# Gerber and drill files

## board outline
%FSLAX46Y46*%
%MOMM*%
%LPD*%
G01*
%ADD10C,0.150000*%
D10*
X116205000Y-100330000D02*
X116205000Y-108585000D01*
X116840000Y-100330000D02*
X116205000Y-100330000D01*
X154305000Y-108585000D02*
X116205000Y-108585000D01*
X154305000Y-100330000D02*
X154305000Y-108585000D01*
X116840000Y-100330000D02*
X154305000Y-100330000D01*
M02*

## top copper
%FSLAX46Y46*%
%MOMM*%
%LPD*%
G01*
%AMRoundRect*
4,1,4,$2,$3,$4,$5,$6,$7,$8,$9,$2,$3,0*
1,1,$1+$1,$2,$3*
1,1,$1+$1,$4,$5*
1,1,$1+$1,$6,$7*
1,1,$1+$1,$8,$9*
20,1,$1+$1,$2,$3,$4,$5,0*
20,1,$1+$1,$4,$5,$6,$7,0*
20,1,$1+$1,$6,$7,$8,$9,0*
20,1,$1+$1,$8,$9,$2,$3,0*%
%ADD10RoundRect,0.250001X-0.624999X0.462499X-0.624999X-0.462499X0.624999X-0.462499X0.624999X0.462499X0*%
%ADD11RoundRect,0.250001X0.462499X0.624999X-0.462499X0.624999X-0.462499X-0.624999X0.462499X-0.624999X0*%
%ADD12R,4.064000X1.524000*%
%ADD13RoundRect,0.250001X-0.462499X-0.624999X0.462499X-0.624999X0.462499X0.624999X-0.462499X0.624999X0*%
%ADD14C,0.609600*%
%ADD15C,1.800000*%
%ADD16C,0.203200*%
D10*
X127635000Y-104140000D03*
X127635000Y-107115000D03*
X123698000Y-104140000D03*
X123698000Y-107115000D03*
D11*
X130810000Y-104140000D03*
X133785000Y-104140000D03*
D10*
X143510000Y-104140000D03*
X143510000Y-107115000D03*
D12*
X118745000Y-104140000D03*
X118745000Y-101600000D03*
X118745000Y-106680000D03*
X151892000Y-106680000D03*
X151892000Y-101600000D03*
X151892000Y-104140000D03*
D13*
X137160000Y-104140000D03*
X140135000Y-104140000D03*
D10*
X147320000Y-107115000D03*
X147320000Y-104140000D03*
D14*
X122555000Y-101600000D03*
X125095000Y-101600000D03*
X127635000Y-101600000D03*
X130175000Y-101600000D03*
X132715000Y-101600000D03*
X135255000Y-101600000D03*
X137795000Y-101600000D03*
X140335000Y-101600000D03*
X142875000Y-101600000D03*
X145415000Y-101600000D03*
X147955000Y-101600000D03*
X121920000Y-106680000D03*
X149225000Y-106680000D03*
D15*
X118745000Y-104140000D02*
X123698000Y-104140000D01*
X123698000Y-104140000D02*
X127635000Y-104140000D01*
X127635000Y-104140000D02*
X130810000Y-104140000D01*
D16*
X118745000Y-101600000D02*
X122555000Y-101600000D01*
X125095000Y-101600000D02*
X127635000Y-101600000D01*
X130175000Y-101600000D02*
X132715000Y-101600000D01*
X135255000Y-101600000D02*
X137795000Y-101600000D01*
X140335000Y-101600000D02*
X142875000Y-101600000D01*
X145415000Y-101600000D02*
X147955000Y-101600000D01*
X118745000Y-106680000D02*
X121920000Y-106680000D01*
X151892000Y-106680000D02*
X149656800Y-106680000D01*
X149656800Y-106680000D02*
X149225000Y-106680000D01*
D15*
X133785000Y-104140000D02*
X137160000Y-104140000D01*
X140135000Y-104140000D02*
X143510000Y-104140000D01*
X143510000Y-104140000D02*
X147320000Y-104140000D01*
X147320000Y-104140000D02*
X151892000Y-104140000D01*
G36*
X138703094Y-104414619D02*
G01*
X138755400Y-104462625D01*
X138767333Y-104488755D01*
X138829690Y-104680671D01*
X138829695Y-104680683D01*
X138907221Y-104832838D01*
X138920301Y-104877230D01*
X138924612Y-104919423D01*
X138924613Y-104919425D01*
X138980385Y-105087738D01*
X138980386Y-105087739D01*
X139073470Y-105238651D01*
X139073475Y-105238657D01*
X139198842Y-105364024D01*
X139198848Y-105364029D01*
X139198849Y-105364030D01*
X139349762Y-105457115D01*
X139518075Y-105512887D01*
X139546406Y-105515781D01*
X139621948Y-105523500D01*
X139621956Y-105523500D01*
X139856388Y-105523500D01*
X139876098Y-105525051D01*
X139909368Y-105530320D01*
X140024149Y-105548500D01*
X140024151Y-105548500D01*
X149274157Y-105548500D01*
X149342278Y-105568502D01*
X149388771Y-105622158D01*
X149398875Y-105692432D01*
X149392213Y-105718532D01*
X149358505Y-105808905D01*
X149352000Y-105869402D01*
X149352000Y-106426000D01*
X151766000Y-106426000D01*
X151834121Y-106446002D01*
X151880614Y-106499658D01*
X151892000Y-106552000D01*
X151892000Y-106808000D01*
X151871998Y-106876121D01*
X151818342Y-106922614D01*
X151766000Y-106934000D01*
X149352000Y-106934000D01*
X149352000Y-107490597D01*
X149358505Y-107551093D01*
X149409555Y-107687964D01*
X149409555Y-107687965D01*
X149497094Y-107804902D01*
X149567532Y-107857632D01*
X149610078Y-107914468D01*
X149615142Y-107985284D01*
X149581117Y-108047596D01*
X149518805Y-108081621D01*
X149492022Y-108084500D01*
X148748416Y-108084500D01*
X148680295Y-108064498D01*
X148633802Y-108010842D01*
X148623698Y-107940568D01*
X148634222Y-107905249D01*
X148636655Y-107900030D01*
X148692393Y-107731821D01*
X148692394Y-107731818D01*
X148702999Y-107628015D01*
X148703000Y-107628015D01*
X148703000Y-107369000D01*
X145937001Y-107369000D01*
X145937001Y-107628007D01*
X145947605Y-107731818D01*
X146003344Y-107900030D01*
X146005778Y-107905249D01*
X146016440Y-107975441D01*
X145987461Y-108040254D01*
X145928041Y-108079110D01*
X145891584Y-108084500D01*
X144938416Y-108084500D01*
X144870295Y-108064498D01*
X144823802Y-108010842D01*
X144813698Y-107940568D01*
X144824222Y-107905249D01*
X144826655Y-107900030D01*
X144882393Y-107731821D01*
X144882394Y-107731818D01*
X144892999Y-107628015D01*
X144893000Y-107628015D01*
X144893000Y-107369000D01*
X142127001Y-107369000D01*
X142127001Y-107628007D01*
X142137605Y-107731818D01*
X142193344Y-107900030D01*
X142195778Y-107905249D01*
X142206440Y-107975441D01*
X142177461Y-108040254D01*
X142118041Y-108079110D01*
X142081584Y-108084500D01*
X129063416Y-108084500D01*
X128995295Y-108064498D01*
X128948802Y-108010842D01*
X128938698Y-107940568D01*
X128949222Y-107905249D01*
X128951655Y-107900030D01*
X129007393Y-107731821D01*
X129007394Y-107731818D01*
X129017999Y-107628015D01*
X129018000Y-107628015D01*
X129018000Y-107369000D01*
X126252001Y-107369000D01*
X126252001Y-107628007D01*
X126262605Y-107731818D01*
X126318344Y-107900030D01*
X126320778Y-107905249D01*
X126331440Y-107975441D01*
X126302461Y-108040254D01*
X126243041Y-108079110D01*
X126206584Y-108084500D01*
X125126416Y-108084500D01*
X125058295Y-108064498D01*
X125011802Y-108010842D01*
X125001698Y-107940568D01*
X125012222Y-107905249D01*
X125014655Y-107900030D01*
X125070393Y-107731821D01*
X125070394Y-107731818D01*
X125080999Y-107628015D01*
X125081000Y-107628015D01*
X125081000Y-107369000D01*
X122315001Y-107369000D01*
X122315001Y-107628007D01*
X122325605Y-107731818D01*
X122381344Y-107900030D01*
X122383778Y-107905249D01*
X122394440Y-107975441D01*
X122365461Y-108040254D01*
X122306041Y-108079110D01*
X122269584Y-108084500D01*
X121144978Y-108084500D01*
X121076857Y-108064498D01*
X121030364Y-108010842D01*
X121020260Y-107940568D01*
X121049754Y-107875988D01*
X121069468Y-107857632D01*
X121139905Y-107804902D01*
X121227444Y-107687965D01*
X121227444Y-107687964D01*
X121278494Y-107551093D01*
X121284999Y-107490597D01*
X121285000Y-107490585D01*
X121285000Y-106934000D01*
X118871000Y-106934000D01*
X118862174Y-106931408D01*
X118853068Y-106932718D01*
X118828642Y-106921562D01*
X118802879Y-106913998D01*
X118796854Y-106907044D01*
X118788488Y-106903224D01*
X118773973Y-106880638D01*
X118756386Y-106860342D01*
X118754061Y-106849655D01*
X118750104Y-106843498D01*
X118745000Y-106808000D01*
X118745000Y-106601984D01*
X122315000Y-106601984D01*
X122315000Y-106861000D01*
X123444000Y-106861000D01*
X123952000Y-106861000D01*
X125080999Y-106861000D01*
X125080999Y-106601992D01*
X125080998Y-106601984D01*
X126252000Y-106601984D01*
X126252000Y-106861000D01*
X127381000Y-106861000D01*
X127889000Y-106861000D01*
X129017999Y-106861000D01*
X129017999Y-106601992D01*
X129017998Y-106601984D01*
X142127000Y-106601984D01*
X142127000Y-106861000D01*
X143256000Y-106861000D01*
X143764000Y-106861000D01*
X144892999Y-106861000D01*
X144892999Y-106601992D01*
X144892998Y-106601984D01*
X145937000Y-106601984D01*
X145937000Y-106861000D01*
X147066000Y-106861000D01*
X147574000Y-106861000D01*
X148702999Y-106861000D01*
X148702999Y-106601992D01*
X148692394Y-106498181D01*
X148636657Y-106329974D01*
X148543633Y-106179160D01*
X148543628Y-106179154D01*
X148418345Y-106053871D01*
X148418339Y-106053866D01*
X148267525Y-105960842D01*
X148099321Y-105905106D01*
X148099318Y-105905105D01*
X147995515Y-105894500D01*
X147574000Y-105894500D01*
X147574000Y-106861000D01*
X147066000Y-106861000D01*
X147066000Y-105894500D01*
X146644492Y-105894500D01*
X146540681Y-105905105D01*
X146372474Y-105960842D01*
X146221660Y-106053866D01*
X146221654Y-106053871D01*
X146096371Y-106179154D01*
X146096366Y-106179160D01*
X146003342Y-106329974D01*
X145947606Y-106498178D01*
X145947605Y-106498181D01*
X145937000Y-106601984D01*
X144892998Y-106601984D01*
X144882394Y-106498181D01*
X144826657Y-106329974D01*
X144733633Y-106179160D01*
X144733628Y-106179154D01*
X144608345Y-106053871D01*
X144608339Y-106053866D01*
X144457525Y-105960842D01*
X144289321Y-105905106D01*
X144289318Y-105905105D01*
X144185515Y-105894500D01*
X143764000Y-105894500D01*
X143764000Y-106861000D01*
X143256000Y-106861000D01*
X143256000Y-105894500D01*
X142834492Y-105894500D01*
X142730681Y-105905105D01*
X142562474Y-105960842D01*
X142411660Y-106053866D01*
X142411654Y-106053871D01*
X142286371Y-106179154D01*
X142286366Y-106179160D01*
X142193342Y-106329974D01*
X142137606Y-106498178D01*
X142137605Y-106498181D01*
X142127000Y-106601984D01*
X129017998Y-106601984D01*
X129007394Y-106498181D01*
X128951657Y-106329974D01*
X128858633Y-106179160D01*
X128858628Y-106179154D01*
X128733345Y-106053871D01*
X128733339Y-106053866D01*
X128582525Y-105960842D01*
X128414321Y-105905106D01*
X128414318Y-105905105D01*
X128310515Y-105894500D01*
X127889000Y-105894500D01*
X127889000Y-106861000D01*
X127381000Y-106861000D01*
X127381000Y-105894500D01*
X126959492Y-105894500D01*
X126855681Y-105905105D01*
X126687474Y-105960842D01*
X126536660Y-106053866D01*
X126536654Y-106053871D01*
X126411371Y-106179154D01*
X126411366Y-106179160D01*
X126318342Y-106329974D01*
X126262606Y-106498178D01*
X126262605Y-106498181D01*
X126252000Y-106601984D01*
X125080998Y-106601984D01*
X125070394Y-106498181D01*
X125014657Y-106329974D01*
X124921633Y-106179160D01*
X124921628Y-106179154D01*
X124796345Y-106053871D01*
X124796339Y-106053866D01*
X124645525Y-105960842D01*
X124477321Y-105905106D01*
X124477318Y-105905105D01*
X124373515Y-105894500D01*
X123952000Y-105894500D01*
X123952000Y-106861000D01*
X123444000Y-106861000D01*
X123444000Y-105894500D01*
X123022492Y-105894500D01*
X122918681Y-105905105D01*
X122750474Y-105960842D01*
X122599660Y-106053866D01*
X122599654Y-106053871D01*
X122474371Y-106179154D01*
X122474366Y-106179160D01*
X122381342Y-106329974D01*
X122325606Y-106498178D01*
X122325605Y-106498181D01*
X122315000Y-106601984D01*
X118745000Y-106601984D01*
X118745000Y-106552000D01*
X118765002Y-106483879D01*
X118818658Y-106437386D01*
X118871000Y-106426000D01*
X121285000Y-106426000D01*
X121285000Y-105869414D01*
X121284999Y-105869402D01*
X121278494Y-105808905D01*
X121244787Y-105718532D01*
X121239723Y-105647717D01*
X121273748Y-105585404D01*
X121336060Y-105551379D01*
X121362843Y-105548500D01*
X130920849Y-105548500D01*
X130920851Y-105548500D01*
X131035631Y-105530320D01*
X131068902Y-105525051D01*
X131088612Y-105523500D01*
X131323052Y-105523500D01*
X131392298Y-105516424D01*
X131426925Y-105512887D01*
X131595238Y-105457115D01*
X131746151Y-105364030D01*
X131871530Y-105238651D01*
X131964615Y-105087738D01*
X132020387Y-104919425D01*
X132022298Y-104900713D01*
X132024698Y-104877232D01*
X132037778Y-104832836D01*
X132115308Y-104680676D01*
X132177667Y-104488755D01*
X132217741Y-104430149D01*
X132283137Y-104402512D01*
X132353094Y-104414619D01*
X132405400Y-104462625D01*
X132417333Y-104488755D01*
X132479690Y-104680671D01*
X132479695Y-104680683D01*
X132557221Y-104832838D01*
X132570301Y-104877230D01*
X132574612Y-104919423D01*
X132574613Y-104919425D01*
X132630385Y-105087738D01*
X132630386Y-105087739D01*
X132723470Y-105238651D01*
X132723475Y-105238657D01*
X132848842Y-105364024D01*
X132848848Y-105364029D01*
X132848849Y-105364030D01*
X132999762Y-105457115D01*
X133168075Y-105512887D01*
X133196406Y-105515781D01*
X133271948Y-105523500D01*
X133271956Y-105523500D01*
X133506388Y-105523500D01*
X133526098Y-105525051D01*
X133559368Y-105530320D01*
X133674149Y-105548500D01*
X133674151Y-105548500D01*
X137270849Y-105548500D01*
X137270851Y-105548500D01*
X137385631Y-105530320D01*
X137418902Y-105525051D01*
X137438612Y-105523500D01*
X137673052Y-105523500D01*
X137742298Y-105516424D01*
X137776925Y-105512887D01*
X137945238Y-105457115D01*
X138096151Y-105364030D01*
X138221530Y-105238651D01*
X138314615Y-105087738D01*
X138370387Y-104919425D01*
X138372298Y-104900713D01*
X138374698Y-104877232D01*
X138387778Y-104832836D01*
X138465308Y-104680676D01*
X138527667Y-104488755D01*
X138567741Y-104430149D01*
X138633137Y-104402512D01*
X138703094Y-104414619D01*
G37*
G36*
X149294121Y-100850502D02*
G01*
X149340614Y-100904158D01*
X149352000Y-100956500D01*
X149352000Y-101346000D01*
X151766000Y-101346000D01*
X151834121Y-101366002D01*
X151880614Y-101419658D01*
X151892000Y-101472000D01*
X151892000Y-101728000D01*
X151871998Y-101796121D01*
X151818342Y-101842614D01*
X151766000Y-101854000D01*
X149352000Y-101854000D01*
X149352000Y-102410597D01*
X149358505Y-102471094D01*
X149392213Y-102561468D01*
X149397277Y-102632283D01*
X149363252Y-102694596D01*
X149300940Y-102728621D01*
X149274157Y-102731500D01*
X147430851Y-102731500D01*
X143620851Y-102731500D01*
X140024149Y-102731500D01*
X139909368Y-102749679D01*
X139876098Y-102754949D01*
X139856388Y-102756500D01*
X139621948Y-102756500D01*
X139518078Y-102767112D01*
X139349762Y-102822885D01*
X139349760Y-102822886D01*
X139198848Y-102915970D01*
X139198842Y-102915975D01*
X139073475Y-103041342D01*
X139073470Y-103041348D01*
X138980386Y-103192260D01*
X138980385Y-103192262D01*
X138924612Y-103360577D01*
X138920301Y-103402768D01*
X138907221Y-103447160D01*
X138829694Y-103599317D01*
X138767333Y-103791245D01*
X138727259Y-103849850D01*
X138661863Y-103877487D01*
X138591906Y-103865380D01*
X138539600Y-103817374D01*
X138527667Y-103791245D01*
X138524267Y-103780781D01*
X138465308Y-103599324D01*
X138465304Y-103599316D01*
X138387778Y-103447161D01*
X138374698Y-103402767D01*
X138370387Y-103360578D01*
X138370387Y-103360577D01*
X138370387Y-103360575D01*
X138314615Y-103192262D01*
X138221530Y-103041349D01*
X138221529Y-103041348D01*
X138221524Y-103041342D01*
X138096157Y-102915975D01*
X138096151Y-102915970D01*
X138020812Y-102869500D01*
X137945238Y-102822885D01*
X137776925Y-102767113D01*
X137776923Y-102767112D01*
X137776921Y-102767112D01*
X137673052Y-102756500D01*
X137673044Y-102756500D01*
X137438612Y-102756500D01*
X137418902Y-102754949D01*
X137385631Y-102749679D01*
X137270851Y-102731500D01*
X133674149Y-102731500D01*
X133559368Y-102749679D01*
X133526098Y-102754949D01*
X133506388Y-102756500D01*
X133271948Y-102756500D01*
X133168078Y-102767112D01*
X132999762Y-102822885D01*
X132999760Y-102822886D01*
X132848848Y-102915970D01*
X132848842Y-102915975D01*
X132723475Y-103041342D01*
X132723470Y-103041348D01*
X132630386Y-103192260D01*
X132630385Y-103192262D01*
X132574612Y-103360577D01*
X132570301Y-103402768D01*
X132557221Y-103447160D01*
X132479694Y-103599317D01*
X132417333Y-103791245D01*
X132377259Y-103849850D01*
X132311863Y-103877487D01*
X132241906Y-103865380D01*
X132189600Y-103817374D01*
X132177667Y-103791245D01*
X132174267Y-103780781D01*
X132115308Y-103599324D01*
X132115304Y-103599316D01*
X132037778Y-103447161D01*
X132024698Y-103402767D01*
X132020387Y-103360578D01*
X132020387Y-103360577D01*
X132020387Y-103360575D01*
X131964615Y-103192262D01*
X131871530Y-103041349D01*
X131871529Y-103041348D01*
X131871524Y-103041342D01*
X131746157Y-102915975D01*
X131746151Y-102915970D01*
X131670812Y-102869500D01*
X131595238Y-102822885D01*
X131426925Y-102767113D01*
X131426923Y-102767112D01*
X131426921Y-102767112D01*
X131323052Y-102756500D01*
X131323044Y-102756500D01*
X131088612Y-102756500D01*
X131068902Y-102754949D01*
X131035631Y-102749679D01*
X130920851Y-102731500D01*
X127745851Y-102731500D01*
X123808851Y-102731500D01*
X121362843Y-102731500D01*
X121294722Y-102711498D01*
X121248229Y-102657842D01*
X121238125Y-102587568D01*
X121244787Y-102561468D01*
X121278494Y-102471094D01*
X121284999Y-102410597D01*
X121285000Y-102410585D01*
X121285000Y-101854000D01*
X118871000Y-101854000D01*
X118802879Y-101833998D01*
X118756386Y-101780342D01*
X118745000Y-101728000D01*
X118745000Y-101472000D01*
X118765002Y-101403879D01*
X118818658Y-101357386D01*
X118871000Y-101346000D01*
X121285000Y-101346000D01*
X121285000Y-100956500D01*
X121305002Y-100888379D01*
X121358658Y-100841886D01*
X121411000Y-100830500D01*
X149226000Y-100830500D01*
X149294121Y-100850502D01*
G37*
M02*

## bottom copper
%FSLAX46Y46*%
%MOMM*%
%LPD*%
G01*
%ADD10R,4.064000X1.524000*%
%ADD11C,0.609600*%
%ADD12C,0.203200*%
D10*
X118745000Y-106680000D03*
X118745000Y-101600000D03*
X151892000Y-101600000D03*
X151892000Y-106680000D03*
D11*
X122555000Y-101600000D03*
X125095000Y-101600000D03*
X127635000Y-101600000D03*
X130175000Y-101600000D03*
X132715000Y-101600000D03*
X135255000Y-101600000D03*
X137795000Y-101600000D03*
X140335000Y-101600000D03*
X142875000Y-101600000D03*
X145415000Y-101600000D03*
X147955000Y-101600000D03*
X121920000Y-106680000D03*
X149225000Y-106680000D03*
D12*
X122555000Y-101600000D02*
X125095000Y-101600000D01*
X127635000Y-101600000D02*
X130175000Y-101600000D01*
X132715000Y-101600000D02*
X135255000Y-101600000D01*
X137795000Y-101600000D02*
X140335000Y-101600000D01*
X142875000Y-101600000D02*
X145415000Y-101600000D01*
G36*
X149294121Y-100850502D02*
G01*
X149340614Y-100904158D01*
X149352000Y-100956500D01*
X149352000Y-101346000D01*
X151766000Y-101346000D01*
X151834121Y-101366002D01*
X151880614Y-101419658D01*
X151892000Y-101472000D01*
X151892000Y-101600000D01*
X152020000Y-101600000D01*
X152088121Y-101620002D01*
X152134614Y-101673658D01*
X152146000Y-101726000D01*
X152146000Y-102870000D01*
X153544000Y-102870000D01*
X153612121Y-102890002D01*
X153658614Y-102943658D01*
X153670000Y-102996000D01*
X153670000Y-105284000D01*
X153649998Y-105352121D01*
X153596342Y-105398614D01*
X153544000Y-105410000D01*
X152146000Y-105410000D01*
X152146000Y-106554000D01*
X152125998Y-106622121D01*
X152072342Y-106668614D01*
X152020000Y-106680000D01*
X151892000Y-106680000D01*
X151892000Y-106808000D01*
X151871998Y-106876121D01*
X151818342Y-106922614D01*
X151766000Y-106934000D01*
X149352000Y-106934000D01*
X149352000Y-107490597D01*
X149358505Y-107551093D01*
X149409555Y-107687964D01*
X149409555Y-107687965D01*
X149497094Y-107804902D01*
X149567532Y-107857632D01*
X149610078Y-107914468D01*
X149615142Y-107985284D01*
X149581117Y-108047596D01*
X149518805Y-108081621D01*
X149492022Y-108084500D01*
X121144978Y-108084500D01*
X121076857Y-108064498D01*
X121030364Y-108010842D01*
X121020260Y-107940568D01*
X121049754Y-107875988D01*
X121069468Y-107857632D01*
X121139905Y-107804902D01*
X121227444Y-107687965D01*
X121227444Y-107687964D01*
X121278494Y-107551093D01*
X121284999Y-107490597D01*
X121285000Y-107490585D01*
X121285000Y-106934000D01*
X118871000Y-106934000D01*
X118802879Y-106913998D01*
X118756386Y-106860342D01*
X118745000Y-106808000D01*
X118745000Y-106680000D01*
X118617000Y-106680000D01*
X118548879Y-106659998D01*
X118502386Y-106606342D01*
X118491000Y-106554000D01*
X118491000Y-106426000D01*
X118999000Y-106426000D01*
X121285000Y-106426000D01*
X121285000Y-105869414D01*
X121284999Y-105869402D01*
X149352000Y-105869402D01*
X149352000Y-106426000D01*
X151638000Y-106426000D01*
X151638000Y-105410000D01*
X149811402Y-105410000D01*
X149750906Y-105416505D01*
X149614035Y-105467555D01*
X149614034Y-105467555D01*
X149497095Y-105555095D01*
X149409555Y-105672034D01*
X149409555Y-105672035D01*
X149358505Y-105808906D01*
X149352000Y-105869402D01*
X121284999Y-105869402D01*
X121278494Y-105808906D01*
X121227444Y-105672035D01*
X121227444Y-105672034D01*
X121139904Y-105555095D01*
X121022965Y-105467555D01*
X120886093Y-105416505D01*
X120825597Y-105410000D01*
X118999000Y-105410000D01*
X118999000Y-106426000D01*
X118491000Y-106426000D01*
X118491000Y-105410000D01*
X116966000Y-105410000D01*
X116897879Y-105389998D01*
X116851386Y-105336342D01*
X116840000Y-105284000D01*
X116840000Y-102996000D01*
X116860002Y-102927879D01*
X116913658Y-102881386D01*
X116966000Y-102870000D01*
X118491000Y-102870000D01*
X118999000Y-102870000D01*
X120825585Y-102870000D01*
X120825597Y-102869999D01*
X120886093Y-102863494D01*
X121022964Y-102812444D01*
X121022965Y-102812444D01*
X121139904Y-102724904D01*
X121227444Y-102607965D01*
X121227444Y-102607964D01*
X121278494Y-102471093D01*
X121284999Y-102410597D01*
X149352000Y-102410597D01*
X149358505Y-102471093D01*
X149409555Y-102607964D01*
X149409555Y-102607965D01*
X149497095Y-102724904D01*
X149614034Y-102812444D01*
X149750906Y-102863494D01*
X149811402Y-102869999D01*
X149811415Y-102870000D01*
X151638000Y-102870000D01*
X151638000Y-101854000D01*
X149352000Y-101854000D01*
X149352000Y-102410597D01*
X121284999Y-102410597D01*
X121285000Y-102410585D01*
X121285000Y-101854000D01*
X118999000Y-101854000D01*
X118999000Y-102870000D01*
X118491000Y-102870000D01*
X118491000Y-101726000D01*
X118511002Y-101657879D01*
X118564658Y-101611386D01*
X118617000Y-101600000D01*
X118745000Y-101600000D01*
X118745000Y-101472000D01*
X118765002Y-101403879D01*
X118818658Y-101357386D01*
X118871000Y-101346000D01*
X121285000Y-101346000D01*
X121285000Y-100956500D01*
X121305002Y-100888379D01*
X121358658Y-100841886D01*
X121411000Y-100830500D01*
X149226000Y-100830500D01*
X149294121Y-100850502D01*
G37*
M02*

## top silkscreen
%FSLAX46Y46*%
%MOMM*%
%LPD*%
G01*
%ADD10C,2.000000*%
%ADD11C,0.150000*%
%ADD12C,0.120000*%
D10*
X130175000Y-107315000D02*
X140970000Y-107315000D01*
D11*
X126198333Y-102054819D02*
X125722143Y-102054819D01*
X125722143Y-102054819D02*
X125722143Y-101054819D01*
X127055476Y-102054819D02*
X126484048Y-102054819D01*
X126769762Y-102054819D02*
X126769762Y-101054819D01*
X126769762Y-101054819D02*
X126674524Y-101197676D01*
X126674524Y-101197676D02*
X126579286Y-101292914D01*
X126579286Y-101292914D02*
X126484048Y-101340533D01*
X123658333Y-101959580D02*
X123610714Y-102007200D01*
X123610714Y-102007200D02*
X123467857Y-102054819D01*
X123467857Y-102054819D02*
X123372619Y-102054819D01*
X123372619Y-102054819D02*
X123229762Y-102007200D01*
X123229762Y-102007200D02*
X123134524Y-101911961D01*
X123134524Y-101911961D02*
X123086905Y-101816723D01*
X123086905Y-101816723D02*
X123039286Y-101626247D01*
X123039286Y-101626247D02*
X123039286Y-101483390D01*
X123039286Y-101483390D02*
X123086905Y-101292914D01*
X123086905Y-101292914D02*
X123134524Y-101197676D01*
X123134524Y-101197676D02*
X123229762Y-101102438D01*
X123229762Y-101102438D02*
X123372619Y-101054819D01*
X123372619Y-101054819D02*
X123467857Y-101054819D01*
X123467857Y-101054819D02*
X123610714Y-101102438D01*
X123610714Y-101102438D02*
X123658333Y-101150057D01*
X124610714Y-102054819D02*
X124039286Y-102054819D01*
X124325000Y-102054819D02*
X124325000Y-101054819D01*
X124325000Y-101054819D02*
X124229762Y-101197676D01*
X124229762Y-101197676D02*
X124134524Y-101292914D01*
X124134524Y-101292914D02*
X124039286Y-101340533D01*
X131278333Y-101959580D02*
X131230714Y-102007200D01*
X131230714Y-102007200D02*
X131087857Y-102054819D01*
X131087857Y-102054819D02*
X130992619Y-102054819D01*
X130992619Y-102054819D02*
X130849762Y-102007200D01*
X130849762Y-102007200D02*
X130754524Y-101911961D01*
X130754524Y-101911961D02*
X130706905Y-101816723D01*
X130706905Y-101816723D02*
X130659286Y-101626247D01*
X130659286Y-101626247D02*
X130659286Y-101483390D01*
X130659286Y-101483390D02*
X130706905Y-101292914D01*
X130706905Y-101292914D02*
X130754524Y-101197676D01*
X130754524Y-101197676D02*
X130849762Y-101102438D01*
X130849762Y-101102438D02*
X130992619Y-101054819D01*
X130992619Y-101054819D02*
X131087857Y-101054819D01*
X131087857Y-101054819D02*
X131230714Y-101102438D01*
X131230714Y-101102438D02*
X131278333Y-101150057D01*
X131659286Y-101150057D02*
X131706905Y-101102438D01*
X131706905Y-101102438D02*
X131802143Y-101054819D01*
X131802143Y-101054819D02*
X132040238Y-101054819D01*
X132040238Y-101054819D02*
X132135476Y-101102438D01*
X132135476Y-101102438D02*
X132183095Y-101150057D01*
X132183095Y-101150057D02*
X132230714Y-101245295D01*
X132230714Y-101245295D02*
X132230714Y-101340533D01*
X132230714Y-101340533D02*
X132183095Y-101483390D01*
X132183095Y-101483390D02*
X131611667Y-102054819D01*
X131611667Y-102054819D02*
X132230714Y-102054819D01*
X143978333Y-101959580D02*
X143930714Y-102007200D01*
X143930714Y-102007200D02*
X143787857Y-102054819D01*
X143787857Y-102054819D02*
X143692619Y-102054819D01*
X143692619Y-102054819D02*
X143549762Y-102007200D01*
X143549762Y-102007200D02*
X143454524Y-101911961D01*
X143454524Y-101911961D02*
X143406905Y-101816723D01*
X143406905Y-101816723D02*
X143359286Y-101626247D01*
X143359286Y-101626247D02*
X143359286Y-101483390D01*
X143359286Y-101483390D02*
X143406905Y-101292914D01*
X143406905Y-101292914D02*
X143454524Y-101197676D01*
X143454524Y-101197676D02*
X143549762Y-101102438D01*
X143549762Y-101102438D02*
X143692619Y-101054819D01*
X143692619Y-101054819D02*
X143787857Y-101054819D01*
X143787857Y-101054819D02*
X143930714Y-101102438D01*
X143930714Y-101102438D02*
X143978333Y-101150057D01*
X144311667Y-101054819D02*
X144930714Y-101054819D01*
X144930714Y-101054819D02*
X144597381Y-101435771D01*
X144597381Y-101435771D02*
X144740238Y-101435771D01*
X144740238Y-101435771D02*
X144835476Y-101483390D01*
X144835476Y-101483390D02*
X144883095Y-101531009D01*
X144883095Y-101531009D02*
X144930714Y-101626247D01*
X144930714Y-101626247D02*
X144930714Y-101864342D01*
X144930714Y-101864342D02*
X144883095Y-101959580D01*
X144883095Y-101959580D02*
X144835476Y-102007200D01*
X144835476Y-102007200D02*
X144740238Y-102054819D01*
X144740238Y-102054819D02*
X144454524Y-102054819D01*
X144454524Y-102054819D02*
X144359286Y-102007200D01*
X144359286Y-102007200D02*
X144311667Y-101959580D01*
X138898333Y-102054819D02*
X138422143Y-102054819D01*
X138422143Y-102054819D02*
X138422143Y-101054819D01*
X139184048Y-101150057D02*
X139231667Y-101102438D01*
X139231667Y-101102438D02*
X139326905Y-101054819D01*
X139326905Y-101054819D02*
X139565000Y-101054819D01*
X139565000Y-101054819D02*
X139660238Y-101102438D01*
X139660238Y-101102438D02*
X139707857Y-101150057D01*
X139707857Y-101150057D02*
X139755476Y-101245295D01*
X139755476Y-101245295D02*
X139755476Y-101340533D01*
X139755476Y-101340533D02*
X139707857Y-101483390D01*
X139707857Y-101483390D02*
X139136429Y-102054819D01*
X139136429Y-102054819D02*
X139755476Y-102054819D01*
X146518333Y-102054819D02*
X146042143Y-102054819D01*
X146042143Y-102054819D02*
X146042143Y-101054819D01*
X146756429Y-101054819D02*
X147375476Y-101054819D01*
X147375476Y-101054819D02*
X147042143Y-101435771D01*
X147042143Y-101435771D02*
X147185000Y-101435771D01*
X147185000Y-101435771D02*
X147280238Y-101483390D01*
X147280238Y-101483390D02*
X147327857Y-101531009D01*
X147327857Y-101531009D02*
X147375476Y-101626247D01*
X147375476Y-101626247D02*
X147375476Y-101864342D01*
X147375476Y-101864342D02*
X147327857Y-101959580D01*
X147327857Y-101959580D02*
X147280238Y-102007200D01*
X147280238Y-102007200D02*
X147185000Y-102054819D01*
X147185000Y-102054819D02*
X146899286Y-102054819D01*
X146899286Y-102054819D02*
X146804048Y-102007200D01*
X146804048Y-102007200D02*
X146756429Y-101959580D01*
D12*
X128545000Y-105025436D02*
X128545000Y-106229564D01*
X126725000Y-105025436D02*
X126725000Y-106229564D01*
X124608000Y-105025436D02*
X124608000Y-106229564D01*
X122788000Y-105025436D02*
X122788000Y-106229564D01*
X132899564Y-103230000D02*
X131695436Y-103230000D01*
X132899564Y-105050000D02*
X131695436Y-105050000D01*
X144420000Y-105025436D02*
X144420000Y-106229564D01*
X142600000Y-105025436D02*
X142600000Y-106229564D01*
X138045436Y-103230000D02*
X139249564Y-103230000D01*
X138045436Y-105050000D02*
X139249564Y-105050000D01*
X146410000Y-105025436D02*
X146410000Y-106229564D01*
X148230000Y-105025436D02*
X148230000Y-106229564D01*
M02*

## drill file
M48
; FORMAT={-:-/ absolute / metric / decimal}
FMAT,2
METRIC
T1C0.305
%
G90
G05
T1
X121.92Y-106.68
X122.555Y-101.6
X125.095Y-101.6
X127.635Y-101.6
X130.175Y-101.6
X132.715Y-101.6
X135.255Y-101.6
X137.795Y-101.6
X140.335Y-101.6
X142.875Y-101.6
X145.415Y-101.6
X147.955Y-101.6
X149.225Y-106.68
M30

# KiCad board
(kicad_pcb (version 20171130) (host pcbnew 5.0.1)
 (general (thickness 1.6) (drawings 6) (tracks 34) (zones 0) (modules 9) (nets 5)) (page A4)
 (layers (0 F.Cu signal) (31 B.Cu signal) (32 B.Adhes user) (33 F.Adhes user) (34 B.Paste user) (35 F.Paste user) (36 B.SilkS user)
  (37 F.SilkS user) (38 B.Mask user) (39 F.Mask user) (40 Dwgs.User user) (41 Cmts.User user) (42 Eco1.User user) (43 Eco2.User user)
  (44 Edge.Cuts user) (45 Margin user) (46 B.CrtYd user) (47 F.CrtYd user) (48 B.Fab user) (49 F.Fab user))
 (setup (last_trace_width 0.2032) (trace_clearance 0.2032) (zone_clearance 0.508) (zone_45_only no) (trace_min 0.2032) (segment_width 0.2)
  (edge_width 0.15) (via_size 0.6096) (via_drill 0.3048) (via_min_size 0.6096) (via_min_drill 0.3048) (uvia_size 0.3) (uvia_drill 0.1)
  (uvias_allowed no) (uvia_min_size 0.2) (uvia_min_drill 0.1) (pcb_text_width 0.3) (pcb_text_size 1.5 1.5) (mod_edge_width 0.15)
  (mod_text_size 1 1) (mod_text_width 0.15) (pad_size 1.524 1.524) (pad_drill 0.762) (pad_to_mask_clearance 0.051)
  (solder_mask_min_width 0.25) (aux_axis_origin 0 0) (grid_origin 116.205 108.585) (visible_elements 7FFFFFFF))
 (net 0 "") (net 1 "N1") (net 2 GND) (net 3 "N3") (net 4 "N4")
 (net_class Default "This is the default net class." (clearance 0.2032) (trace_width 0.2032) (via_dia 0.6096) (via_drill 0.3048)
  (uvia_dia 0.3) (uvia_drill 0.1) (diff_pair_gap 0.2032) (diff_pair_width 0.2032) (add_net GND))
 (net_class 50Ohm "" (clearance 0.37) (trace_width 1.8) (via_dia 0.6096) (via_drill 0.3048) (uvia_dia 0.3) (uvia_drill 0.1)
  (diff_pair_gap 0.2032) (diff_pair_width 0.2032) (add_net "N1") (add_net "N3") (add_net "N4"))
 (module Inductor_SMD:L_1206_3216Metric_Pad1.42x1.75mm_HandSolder (layer F.Cu) (at 127.635 105.6275 270)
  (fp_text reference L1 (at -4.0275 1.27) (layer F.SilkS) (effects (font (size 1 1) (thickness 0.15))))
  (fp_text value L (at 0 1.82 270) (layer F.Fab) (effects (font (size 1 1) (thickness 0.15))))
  (fp_line (start -0.602064 -0.91) (end 0.602064 -0.91) (layer F.SilkS) (width 0.12))
  (fp_line (start -0.602064 0.91) (end 0.602064 0.91) (layer F.SilkS) (width 0.12))
  (pad 1 smd roundrect (at -1.4875 0 270) (size 1.425 1.75) (layers F.Cu F.Paste F.Mask) (roundrect_rratio 0.175439) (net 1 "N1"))
  (pad 2 smd roundrect (at 1.4875 0 270) (size 1.425 1.75) (layers F.Cu F.Paste F.Mask) (roundrect_rratio 0.175439) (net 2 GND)))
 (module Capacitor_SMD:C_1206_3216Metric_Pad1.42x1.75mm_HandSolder (layer F.Cu) (at 123.698 105.6275 270)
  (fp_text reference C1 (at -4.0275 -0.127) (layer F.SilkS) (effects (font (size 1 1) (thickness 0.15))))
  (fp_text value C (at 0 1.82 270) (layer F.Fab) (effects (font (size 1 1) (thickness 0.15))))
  (fp_line (start -0.602064 -0.91) (end 0.602064 -0.91) (layer F.SilkS) (width 0.12))
  (fp_line (start -0.602064 0.91) (end 0.602064 0.91) (layer F.SilkS) (width 0.12))
  (pad 1 smd roundrect (at -1.4875 0 270) (size 1.425 1.75) (layers F.Cu F.Paste F.Mask) (roundrect_rratio 0.175439) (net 1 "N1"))
  (pad 2 smd roundrect (at 1.4875 0 270) (size 1.425 1.75) (layers F.Cu F.Paste F.Mask) (roundrect_rratio 0.175439) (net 2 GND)))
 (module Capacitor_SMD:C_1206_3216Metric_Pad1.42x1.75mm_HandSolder (layer F.Cu) (at 132.2975 104.14 180)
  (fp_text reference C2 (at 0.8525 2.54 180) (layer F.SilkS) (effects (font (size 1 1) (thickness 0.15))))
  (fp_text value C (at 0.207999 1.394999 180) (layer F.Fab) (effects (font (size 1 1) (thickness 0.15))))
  (fp_line (start -0.602064 0.91) (end 0.602064 0.91) (layer F.SilkS) (width 0.12))
  (fp_line (start -0.602064 -0.91) (end 0.602064 -0.91) (layer F.SilkS) (width 0.12))
  (pad 2 smd roundrect (at 1.4875 0 180) (size 1.425 1.75) (layers F.Cu F.Paste F.Mask) (roundrect_rratio 0.175439) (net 1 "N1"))
  (pad 1 smd roundrect (at -1.4875 0 180) (size 1.425 1.75) (layers F.Cu F.Paste F.Mask) (roundrect_rratio 0.175439) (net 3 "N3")))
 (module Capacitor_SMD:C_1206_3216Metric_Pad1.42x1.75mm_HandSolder (layer F.Cu) (at 143.51 105.6275 270)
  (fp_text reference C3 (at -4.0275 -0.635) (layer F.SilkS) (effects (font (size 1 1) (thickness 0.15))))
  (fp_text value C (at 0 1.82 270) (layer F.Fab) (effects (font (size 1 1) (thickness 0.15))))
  (fp_line (start -0.602064 -0.91) (end 0.602064 -0.91) (layer F.SilkS) (width 0.12))
  (fp_line (start -0.602064 0.91) (end 0.602064 0.91) (layer F.SilkS) (width 0.12))
  (pad 1 smd roundrect (at -1.4875 0 270) (size 1.425 1.75) (layers F.Cu F.Paste F.Mask) (roundrect_rratio 0.175439) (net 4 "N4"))
  (pad 2 smd roundrect (at 1.4875 0 270) (size 1.425 1.75) (layers F.Cu F.Paste F.Mask) (roundrect_rratio 0.175439) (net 2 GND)))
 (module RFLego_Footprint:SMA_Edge (layer F.Cu) (at 116.713 104.14)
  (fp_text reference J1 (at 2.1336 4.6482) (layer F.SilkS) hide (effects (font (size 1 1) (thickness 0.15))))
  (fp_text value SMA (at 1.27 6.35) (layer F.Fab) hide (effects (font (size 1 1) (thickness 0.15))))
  (pad 1 smd rect (at 2.032 0) (size 4.064 1.524) (layers F.Cu F.Mask) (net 1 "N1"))
  (pad 2 smd rect (at 2.032 -2.54) (size 4.064 1.524) (layers F.Cu F.Mask) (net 2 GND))
  (pad 2 smd rect (at 2.032 2.54) (size 4.064 1.524) (layers B.Cu B.Mask) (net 2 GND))
  (pad 2 smd rect (at 2.032 -2.54) (size 4.064 1.524) (layers B.Cu B.Mask) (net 2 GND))
  (pad 2 smd rect (at 2.032 2.54) (size 4.064 1.524) (layers F.Cu F.Mask) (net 2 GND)))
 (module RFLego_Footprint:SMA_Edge (layer F.Cu) (at 149.86 104.14)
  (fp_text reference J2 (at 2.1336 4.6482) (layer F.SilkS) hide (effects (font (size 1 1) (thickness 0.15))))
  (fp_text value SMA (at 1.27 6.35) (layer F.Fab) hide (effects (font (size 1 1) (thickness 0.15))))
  (pad 2 smd rect (at 2.032 2.54) (size 4.064 1.524) (layers F.Cu F.Mask) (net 2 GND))
  (pad 2 smd rect (at 2.032 -2.54) (size 4.064 1.524) (layers B.Cu B.Mask) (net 2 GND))
  (pad 2 smd rect (at 2.032 2.54) (size 4.064 1.524) (layers B.Cu B.Mask) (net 2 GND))
  (pad 2 smd rect (at 2.032 -2.54) (size 4.064 1.524) (layers F.Cu F.Mask) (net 2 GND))
  (pad 1 smd rect (at 2.032 0) (size 4.064 1.524) (layers F.Cu F.Mask) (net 4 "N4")))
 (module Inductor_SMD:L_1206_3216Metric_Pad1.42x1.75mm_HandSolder (layer F.Cu) (at 138.6475 104.14)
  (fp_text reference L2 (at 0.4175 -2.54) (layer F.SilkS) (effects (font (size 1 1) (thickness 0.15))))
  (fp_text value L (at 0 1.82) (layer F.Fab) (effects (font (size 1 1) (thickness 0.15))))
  (fp_line (start -0.602064 -0.91) (end 0.602064 -0.91) (layer F.SilkS) (width 0.12))
  (fp_line (start -0.602064 0.91) (end 0.602064 0.91) (layer F.SilkS) (width 0.12))
  (pad 1 smd roundrect (at -1.4875 0) (size 1.425 1.75) (layers F.Cu F.Paste F.Mask) (roundrect_rratio 0.175439) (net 3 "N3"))
  (pad 2 smd roundrect (at 1.4875 0) (size 1.425 1.75) (layers F.Cu F.Paste F.Mask) (roundrect_rratio 0.175439) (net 4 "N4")))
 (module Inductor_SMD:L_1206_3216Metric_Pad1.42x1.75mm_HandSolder (layer F.Cu) (at 147.32 105.6275 270)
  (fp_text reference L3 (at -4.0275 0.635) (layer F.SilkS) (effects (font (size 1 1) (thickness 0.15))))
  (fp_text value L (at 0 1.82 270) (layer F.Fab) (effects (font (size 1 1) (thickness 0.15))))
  (fp_line (start -0.602064 0.91) (end 0.602064 0.91) (layer F.SilkS) (width 0.12))
  (fp_line (start -0.602064 -0.91) (end 0.602064 -0.91) (layer F.SilkS) (width 0.12))
  (pad 2 smd roundrect (at 1.4875 0 270) (size 1.425 1.75) (layers F.Cu F.Paste F.Mask) (roundrect_rratio 0.175439) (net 2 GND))
  (pad 1 smd roundrect (at -1.4875 0 270) (size 1.425 1.75) (layers F.Cu F.Paste F.Mask) (roundrect_rratio 0.175439) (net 4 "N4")))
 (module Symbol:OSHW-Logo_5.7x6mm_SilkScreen (layer B.Cu) (at 126.365 104.775 180)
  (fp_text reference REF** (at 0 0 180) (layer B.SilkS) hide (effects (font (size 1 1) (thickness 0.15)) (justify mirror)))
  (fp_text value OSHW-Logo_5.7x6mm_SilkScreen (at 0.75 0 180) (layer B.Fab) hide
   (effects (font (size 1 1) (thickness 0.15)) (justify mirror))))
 (gr_line (start 116.205 100.33) (end 116.205 108.585) (layer Edge.Cuts) (width 0.15))
 (gr_line (start 116.84 100.33) (end 116.205 100.33) (layer Edge.Cuts) (width 0.15))
 (gr_line (start 154.305 108.585) (end 116.205 108.585) (layer Edge.Cuts) (width 0.15))
 (gr_line (start 154.305 100.33) (end 154.305 108.585) (layer Edge.Cuts) (width 0.15))
 (gr_line (start 116.84 100.33) (end 154.305 100.33) (layer Edge.Cuts) (width 0.15))
 (gr_line (start 130.175 107.315) (end 140.97 107.315) (layer F.SilkS) (width 2))
 (segment (start 118.745 104.14) (end 123.698 104.14) (width 1.8) (layer F.Cu) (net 1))
 (segment (start 123.698 104.14) (end 127.635 104.14) (width 1.8) (layer F.Cu) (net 1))
 (segment (start 127.635 104.14) (end 130.81 104.14) (width 1.8) (layer F.Cu) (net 1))
 (via (at 122.555 101.6) (size 0.6096) (drill 0.3048) (layers F.Cu B.Cu) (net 2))
 (segment (start 118.745 101.6) (end 122.555 101.6) (width 0.2032) (layer F.Cu) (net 2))
 (via (at 125.095 101.6) (size 0.6096) (drill 0.3048) (layers F.Cu B.Cu) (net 2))
 (segment (start 122.555 101.6) (end 125.095 101.6) (width 0.2032) (layer B.Cu) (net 2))
 (via (at 127.635 101.6) (size 0.6096) (drill 0.3048) (layers F.Cu B.Cu) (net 2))
 (segment (start 125.095 101.6) (end 127.635 101.6) (width 0.2032) (layer F.Cu) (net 2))
 (via (at 130.175 101.6) (size 0.6096) (drill 0.3048) (layers F.Cu B.Cu) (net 2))
 (segment (start 127.635 101.6) (end 130.175 101.6) (width 0.2032) (layer B.Cu) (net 2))
 (via (at 132.715 101.6) (size 0.6096) (drill 0.3048) (layers F.Cu B.Cu) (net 2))
 (segment (start 130.175 101.6) (end 132.715 101.6) (width 0.2032) (layer F.Cu) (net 2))
 (via (at 135.255 101.6) (size 0.6096) (drill 0.3048) (layers F.Cu B.Cu) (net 2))
 (segment (start 132.715 101.6) (end 135.255 101.6) (width 0.2032) (layer B.Cu) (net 2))
 (via (at 137.795 101.6) (size 0.6096) (drill 0.3048) (layers F.Cu B.Cu) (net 2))
 (segment (start 135.255 101.6) (end 137.795 101.6) (width 0.2032) (layer F.Cu) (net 2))
 (via (at 140.335 101.6) (size 0.6096) (drill 0.3048) (layers F.Cu B.Cu) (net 2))
 (segment (start 137.795 101.6) (end 140.335 101.6) (width 0.2032) (layer B.Cu) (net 2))
 (via (at 142.875 101.6) (size 0.6096) (drill 0.3048) (layers F.Cu B.Cu) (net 2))
 (segment (start 140.335 101.6) (end 142.875 101.6) (width 0.2032) (layer F.Cu) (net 2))
 (via (at 145.415 101.6) (size 0.6096) (drill 0.3048) (layers F.Cu B.Cu) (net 2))
 (segment (start 142.875 101.6) (end 145.415 101.6) (width 0.2032) (layer B.Cu) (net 2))
 (via (at 147.955 101.6) (size 0.6096) (drill 0.3048) (layers F.Cu B.Cu) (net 2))
 (segment (start 145.415 101.6) (end 147.955 101.6) (width 0.2032) (layer F.Cu) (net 2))
 (via (at 121.92 106.68) (size 0.6096) (drill 0.3048) (layers F.Cu B.Cu) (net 2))
 (segment (start 118.745 106.68) (end 121.92 106.68) (width 0.2032) (layer F.Cu) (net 2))
 (via (at 149.225 106.68) (size 0.6096) (drill 0.3048) (layers F.Cu B.Cu) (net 2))
 (segment (start 151.892 106.68) (end 149.6568 106.68) (width 0.2032) (layer F.Cu) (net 2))
 (segment (start 149.6568 106.68) (end 149.225 106.68) (width 0.2032) (layer F.Cu) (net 2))
 (segment (start 133.785 104.14) (end 137.16 104.14) (width 1.8) (layer F.Cu) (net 3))
 (segment (start 140.135 104.14) (end 143.51 104.14) (width 1.8) (layer F.Cu) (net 4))
 (segment (start 143.51 104.14) (end 147.32 104.14) (width 1.8) (layer F.Cu) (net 4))
 (segment (start 147.32 104.14) (end 151.892 104.14) (width 1.8) (layer F.Cu) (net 4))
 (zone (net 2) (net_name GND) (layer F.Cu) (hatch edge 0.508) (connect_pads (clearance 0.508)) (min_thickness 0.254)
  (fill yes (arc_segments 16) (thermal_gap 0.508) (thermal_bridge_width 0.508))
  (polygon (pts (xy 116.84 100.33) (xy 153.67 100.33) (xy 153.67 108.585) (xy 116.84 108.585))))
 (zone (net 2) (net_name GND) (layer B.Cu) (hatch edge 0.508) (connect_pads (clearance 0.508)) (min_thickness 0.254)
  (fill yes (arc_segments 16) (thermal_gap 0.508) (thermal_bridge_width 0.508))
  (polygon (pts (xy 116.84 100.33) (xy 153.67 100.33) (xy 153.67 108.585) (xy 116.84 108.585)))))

